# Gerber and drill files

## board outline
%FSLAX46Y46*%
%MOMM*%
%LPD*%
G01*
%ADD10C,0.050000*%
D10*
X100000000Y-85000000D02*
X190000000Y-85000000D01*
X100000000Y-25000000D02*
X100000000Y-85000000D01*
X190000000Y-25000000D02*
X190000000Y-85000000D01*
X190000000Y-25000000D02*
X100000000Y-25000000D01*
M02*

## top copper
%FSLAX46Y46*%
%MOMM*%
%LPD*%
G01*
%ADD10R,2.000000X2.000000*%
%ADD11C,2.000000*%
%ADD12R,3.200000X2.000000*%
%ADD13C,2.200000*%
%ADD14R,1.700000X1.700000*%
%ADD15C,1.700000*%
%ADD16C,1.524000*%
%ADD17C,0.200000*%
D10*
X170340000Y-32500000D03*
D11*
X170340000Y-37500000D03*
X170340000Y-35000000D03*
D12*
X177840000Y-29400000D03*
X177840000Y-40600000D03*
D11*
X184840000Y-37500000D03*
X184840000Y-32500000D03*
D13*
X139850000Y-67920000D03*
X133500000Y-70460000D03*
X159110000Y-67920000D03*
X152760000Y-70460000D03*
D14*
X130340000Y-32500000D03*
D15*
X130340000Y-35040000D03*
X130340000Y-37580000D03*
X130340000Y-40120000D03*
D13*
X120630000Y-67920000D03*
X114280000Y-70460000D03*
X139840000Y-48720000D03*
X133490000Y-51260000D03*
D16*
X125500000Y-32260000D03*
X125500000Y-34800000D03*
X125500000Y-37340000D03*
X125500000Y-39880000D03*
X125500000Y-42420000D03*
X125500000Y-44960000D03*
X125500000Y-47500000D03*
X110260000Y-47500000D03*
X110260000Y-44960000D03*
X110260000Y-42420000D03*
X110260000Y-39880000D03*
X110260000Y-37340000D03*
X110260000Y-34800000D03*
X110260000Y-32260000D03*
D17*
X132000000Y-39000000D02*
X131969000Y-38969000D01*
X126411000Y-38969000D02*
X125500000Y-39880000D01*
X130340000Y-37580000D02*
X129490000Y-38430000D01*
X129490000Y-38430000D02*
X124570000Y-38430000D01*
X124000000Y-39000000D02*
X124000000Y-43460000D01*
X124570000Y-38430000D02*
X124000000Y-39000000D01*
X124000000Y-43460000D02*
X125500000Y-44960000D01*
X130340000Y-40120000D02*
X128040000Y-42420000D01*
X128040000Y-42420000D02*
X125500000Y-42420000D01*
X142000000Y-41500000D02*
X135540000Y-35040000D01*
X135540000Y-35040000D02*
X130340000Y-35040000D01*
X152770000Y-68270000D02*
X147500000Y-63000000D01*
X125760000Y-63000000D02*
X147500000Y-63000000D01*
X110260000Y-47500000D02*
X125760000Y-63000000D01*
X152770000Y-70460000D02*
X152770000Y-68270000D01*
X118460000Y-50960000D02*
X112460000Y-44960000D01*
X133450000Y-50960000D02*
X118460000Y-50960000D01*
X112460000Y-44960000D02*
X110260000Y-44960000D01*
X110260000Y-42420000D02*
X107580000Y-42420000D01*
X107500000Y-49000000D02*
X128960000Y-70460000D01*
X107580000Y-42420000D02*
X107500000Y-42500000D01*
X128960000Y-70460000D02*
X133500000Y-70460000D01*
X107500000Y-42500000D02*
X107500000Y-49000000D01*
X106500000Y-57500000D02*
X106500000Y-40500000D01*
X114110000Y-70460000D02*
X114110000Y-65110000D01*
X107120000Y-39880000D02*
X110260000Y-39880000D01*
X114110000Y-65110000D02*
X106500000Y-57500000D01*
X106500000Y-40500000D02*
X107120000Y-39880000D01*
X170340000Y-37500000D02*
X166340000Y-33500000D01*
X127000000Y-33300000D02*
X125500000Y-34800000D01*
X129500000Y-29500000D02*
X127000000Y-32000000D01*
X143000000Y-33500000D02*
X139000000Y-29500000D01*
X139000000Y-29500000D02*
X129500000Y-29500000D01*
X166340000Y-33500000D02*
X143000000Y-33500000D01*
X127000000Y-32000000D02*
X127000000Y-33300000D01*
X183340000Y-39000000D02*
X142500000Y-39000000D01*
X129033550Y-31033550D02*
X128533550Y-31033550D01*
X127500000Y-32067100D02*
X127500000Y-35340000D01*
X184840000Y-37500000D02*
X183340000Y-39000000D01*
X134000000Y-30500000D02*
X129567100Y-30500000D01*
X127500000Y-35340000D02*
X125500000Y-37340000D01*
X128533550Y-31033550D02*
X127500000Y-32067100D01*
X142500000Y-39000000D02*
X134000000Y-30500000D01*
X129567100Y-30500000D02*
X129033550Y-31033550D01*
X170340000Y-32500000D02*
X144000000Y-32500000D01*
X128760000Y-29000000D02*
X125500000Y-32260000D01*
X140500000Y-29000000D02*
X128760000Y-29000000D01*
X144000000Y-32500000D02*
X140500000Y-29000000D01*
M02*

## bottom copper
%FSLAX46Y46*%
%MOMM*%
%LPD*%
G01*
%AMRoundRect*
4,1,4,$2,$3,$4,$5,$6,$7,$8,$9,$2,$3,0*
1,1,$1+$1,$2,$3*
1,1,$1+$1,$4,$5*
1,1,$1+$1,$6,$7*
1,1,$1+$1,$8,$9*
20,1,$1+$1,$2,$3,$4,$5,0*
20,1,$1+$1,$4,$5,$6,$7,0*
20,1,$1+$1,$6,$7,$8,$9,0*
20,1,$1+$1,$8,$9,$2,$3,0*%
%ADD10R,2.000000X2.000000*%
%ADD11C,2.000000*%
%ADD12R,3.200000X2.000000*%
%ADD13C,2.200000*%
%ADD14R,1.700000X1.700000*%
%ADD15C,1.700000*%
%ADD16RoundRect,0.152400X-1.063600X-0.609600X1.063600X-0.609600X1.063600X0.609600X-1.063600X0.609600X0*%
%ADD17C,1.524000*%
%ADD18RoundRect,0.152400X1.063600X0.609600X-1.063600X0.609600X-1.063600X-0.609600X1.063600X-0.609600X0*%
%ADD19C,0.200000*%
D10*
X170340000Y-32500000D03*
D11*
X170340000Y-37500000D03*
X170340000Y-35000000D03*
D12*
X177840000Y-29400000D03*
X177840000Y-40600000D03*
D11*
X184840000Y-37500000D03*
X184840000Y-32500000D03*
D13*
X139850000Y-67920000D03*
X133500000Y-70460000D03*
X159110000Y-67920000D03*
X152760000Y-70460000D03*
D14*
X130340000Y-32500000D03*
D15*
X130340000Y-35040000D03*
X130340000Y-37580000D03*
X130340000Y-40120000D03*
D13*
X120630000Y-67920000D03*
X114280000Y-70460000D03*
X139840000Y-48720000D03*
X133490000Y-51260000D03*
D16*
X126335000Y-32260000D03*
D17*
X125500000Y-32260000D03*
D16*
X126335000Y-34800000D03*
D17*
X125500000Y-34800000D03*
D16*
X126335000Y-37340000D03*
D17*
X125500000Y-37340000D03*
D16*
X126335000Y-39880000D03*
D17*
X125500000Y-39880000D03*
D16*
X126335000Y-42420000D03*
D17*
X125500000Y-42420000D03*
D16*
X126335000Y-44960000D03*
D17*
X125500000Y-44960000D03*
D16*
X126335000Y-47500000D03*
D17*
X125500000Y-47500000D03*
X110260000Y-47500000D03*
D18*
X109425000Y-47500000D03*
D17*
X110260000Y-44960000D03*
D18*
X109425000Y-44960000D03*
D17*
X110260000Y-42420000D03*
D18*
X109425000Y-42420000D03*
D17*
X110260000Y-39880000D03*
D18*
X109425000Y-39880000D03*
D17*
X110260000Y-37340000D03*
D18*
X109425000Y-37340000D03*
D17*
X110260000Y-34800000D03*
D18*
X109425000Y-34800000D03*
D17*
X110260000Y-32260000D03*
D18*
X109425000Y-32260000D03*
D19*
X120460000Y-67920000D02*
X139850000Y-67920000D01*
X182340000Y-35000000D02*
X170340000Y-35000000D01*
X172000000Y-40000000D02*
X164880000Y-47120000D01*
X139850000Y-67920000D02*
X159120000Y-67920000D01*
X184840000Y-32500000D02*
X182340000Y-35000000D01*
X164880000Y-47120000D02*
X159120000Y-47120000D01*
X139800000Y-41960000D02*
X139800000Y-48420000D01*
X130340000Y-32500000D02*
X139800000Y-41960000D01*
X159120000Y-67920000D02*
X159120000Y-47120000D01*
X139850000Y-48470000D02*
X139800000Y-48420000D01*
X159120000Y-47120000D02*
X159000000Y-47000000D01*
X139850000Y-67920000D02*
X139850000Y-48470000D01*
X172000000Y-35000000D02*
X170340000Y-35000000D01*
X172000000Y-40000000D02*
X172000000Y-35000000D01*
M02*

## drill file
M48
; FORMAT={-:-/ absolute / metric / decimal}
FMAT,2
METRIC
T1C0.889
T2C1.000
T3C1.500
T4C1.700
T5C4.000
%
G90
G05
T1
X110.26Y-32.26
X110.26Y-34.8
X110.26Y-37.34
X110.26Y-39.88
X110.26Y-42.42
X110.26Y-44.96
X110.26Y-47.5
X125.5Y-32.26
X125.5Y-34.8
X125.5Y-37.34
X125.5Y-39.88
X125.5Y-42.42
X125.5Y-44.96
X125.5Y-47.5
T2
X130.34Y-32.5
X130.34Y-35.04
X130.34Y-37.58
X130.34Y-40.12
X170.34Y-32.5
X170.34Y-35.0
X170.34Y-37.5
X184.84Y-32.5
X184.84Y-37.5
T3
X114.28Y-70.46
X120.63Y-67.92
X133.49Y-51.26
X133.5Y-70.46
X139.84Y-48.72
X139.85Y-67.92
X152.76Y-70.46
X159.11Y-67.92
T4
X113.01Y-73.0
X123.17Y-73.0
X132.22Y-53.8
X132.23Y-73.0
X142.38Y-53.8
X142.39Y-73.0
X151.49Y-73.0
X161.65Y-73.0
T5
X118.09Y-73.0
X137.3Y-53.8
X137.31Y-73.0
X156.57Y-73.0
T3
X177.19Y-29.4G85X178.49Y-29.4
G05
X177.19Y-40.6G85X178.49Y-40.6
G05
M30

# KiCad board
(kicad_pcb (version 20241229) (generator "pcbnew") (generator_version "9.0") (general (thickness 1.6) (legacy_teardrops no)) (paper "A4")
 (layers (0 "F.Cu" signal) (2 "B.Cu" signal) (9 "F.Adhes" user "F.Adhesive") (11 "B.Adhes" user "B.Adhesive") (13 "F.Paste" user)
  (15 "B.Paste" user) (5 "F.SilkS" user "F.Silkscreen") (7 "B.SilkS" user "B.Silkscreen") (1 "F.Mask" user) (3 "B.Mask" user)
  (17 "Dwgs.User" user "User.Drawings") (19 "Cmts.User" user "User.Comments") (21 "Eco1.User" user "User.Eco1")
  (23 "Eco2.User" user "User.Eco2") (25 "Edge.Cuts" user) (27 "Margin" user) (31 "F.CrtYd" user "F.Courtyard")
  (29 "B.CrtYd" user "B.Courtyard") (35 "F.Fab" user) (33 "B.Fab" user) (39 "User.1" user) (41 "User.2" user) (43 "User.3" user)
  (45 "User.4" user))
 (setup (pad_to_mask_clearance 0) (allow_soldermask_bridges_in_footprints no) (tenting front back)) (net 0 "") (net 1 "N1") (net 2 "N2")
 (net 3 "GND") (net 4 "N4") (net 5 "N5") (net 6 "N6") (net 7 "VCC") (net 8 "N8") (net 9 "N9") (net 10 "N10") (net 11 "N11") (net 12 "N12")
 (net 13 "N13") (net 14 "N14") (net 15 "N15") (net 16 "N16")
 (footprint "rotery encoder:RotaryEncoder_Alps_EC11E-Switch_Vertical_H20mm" (layer "F.Cu") (at 170.34 32.5)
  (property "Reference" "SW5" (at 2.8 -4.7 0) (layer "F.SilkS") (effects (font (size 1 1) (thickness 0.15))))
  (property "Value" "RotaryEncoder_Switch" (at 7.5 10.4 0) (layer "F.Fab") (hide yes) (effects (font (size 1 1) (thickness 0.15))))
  (pad "A" thru_hole rect (at 0 0) (size 2 2) (drill 1) (layers "*.Cu" "*.Mask") (remove_unused_layers no) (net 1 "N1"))
  (pad "B" thru_hole circle (at 0 5) (size 2 2) (drill 1) (layers "*.Cu" "*.Mask") (remove_unused_layers no) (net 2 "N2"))
  (pad "C" thru_hole circle (at 0 2.5) (size 2 2) (drill 1) (layers "*.Cu" "*.Mask") (remove_unused_layers no) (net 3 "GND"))
  (pad "MP" thru_hole rect (at 7.5 -3.1) (size 3.2 2) (drill oval 2.8 1.5) (layers "*.Cu" "*.Mask") (remove_unused_layers no))
  (pad "MP" thru_hole rect (at 7.5 8.1) (size 3.2 2) (drill oval 2.8 1.5) (layers "*.Cu" "*.Mask") (remove_unused_layers no))
  (pad "S1" thru_hole circle (at 14.5 5) (size 2 2) (drill 1) (layers "*.Cu" "*.Mask") (remove_unused_layers no) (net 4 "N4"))
  (pad "S2" thru_hole circle (at 14.5 0) (size 2 2) (drill 1) (layers "*.Cu" "*.Mask") (remove_unused_layers no) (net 3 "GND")))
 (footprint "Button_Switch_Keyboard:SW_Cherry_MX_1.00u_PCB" (layer "F.Cu") (at 139.85 67.92)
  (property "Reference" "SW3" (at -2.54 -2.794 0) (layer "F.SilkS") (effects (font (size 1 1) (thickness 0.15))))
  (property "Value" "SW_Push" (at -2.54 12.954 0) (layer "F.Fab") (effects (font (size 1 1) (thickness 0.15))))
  (pad "" np_thru_hole circle (at -7.62 5.08) (size 1.7 1.7) (drill 1.7) (layers "*.Cu" "*.Mask"))
  (pad "" np_thru_hole circle (at -2.54 5.08) (size 4 4) (drill 4) (layers "*.Cu" "*.Mask"))
  (pad "" np_thru_hole circle (at 2.54 5.08) (size 1.7 1.7) (drill 1.7) (layers "*.Cu" "*.Mask"))
  (pad "1" thru_hole circle (at 0 0) (size 2.2 2.2) (drill 1.5) (layers "*.Cu" "*.Mask") (remove_unused_layers no) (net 3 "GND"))
  (pad "2" thru_hole circle (at -6.35 2.54) (size 2.2 2.2) (drill 1.5) (layers "*.Cu" "*.Mask") (remove_unused_layers no) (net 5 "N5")))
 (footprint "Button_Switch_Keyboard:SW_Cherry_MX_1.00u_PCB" (layer "F.Cu") (at 159.11 67.92)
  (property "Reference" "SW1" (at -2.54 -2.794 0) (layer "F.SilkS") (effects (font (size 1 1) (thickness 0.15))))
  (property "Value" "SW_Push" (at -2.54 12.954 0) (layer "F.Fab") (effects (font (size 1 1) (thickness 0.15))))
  (pad "" np_thru_hole circle (at -7.62 5.08) (size 1.7 1.7) (drill 1.7) (layers "*.Cu" "*.Mask"))
  (pad "" np_thru_hole circle (at -2.54 5.08) (size 4 4) (drill 4) (layers "*.Cu" "*.Mask"))
  (pad "" np_thru_hole circle (at 2.54 5.08) (size 1.7 1.7) (drill 1.7) (layers "*.Cu" "*.Mask"))
  (pad "1" thru_hole circle (at 0 0) (size 2.2 2.2) (drill 1.5) (layers "*.Cu" "*.Mask") (remove_unused_layers no) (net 3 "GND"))
  (pad "2" thru_hole circle (at -6.35 2.54) (size 2.2 2.2) (drill 1.5) (layers "*.Cu" "*.Mask") (remove_unused_layers no) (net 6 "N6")))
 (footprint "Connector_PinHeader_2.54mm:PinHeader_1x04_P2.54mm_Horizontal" (layer "F.Cu") (at 130.34 32.5)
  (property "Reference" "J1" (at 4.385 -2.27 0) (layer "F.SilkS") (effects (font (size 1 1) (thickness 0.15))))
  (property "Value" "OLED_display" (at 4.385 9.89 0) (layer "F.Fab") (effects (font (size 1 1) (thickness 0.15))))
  (pad "1" thru_hole rect (at 0 0) (size 1.7 1.7) (drill 1) (layers "*.Cu" "*.Mask") (remove_unused_layers no) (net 3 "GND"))
  (pad "2" thru_hole circle (at 0 2.54) (size 1.7 1.7) (drill 1) (layers "*.Cu" "*.Mask") (remove_unused_layers no) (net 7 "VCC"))
  (pad "3" thru_hole circle (at 0 5.08) (size 1.7 1.7) (drill 1) (layers "*.Cu" "*.Mask") (remove_unused_layers no) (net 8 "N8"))
  (pad "4" thru_hole circle (at 0 7.62) (size 1.7 1.7) (drill 1) (layers "*.Cu" "*.Mask") (remove_unused_layers no) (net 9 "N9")))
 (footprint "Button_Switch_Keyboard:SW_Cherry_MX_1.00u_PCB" (layer "F.Cu") (at 120.63 67.92)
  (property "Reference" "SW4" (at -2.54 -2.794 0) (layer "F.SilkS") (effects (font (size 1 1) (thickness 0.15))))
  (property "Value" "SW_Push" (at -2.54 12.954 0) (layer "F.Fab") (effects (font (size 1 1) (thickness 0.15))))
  (pad "" np_thru_hole circle (at -7.62 5.08) (size 1.7 1.7) (drill 1.7) (layers "*.Cu" "*.Mask"))
  (pad "" np_thru_hole circle (at -2.54 5.08) (size 4 4) (drill 4) (layers "*.Cu" "*.Mask"))
  (pad "" np_thru_hole circle (at 2.54 5.08) (size 1.7 1.7) (drill 1.7) (layers "*.Cu" "*.Mask"))
  (pad "1" thru_hole circle (at 0 0) (size 2.2 2.2) (drill 1.5) (layers "*.Cu" "*.Mask") (remove_unused_layers no) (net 3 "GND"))
  (pad "2" thru_hole circle (at -6.35 2.54) (size 2.2 2.2) (drill 1.5) (layers "*.Cu" "*.Mask") (remove_unused_layers no) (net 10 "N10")))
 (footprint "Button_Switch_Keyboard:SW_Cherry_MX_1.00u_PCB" (layer "F.Cu") (at 139.84 48.72)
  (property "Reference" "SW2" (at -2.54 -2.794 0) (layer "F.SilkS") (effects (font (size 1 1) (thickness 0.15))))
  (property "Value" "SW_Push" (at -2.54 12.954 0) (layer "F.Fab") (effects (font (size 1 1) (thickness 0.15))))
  (pad "" np_thru_hole circle (at -7.62 5.08) (size 1.7 1.7) (drill 1.7) (layers "*.Cu" "*.Mask"))
  (pad "" np_thru_hole circle (at -2.54 5.08) (size 4 4) (drill 4) (layers "*.Cu" "*.Mask"))
  (pad "" np_thru_hole circle (at 2.54 5.08) (size 1.7 1.7) (drill 1.7) (layers "*.Cu" "*.Mask"))
  (pad "1" thru_hole circle (at 0 0) (size 2.2 2.2) (drill 1.5) (layers "*.Cu" "*.Mask") (remove_unused_layers no) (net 3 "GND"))
  (pad "2" thru_hole circle (at -6.35 2.54) (size 2.2 2.2) (drill 1.5) (layers "*.Cu" "*.Mask") (remove_unused_layers no) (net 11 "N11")))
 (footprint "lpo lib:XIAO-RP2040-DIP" (layer "B.Cu") (at 117.88 39.88 180)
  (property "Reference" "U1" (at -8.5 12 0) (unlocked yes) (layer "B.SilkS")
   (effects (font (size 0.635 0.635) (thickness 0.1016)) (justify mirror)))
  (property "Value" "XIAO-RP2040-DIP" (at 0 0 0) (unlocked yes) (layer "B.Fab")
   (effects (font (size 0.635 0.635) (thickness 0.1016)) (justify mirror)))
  (pad "1" smd roundrect (at -8.455 7.62) (size 2.432 1.524) (layers "B.Cu" "B.Mask") (roundrect_rratio 0.1) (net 1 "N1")
   (thermal_bridge_angle 45))
  (pad "1" thru_hole circle (at -7.62 7.62) (size 1.524 1.524) (drill 0.889) (layers "*.Cu" "*.Mask") (remove_unused_layers no) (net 1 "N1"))
  (pad "2" smd roundrect (at -8.455 5.08) (size 2.432 1.524) (layers "B.Cu" "B.Mask") (roundrect_rratio 0.1) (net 2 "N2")
   (thermal_bridge_angle 45))
  (pad "2" thru_hole circle (at -7.62 5.08) (size 1.524 1.524) (drill 0.889) (layers "*.Cu" "*.Mask") (remove_unused_layers no) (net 2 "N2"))
  (pad "3" smd roundrect (at -8.455 2.54) (size 2.432 1.524) (layers "B.Cu" "B.Mask") (roundrect_rratio 0.1) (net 4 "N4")
   (thermal_bridge_angle 45))
  (pad "3" thru_hole circle (at -7.62 2.54) (size 1.524 1.524) (drill 0.889) (layers "*.Cu" "*.Mask") (remove_unused_layers no) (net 4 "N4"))
  (pad "4" smd roundrect (at -8.455 0) (size 2.432 1.524) (layers "B.Cu" "B.Mask") (roundrect_rratio 0.1) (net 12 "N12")
   (thermal_bridge_angle 45))
  (pad "4" thru_hole circle (at -7.62 0) (size 1.524 1.524) (drill 0.889) (layers "*.Cu" "*.Mask") (remove_unused_layers no) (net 12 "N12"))
  (pad "5" smd roundrect (at -8.455 -2.54) (size 2.432 1.524) (layers "B.Cu" "B.Mask") (roundrect_rratio 0.1) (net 9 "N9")
   (thermal_bridge_angle 45))
  (pad "5" thru_hole circle (at -7.62 -2.54) (size 1.524 1.524) (drill 0.889) (layers "*.Cu" "*.Mask") (remove_unused_layers no)
   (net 9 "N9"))
  (pad "6" smd roundrect (at -8.455 -5.08) (size 2.432 1.524) (layers "B.Cu" "B.Mask") (roundrect_rratio 0.1) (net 8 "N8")
   (thermal_bridge_angle 45))
  (pad "6" thru_hole circle (at -7.62 -5.08) (size 1.524 1.524) (drill 0.889) (layers "*.Cu" "*.Mask") (remove_unused_layers no)
   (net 8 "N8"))
  (pad "7" smd roundrect (at -8.455 -7.62) (size 2.432 1.524) (layers "B.Cu" "B.Mask") (roundrect_rratio 0.1) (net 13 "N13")
   (thermal_bridge_angle 45))
  (pad "7" thru_hole circle (at -7.62 -7.62) (size 1.524 1.524) (drill 0.889) (layers "*.Cu" "*.Mask") (remove_unused_layers no)
   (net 13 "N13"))
  (pad "8" thru_hole circle (at 7.62 -7.62 180) (size 1.524 1.524) (drill 0.889) (layers "*.Cu" "*.Mask") (remove_unused_layers no)
   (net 6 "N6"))
  (pad "8" smd roundrect (at 8.455 -7.62 180) (size 2.432 1.524) (layers "B.Cu" "B.Mask") (roundrect_rratio 0.1) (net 6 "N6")
   (thermal_bridge_angle 45))
  (pad "9" thru_hole circle (at 7.62 -5.08 180) (size 1.524 1.524) (drill 0.889) (layers "*.Cu" "*.Mask") (remove_unused_layers no)
   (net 11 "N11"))
  (pad "9" smd roundrect (at 8.455 -5.08 180) (size 2.432 1.524) (layers "B.Cu" "B.Mask") (roundrect_rratio 0.1) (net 11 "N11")
   (thermal_bridge_angle 45))
  (pad "10" thru_hole circle (at 7.62 -2.54 180) (size 1.524 1.524) (drill 0.889) (layers "*.Cu" "*.Mask") (remove_unused_layers no)
   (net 5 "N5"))
  (pad "10" smd roundrect (at 8.455 -2.54 180) (size 2.432 1.524) (layers "B.Cu" "B.Mask") (roundrect_rratio 0.1) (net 5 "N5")
   (thermal_bridge_angle 45))
  (pad "11" thru_hole circle (at 7.62 0 180) (size 1.524 1.524) (drill 0.889) (layers "*.Cu" "*.Mask") (remove_unused_layers no)
   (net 10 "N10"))
  (pad "11" smd roundrect (at 8.455 0 180) (size 2.432 1.524) (layers "B.Cu" "B.Mask") (roundrect_rratio 0.1) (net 10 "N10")
   (thermal_bridge_angle 45))
  (pad "12" thru_hole circle (at 7.62 2.54 180) (size 1.524 1.524) (drill 0.889) (layers "*.Cu" "*.Mask") (remove_unused_layers no)
   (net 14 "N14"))
  (pad "12" smd roundrect (at 8.455 2.54 180) (size 2.432 1.524) (layers "B.Cu" "B.Mask") (roundrect_rratio 0.1) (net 14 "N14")
   (thermal_bridge_angle 45))
  (pad "13" thru_hole circle (at 7.62 5.08 180) (size 1.524 1.524) (drill 0.889) (layers "*.Cu" "*.Mask") (remove_unused_layers no)
   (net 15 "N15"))
  (pad "13" smd roundrect (at 8.455 5.08 180) (size 2.432 1.524) (layers "B.Cu" "B.Mask") (roundrect_rratio 0.1) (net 15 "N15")
   (thermal_bridge_angle 45))
  (pad "14" thru_hole circle (at 7.62 7.62 180) (size 1.524 1.524) (drill 0.889) (layers "*.Cu" "*.Mask") (remove_unused_layers no)
   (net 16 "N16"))
  (pad "14" smd roundrect (at 8.455 7.62 180) (size 2.432 1.524) (layers "B.Cu" "B.Mask") (roundrect_rratio 0.1) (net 16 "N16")
   (thermal_bridge_angle 45)))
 (gr_line (start 100 85) (end 190 85) (stroke (width 0.05) (type default)) (layer "Edge.Cuts"))
 (gr_line (start 100 25) (end 100 85) (stroke (width 0.05) (type default)) (layer "Edge.Cuts"))
 (gr_line (start 190 25) (end 190 85) (stroke (width 0.05) (type default)) (layer "Edge.Cuts"))
 (gr_line (start 190 25) (end 100 25) (stroke (width 0.05) (type default)) (layer "Edge.Cuts"))
 (segment (start 132 39) (end 131.969 38.969) (width 0.2) (layer "F.Cu") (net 12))
 (segment (start 126.411 38.969) (end 125.5 39.88) (width 0.2) (layer "F.Cu") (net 12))
 (segment (start 120.46 67.92) (end 139.85 67.92) (width 0.2) (layer "B.Cu") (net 3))
 (segment (start 182.34 35) (end 170.34 35) (width 0.2) (layer "B.Cu") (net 3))
 (segment (start 172 40) (end 164.88 47.12) (width 0.2) (layer "B.Cu") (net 3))
 (segment (start 139.85 67.92) (end 159.12 67.92) (width 0.2) (layer "B.Cu") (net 3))
 (segment (start 184.84 32.5) (end 182.34 35) (width 0.2) (layer "B.Cu") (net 3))
 (segment (start 164.88 47.12) (end 159.12 47.12) (width 0.2) (layer "B.Cu") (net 3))
 (segment (start 139.8 41.96) (end 139.8 48.42) (width 0.2) (layer "B.Cu") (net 3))
 (segment (start 130.34 32.5) (end 139.8 41.96) (width 0.2) (layer "B.Cu") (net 3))
 (segment (start 159.12 67.92) (end 159.12 47.12) (width 0.2) (layer "B.Cu") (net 3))
 (segment (start 139.85 48.47) (end 139.8 48.42) (width 0.2) (layer "B.Cu") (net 3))
 (segment (start 159.12 47.12) (end 159 47) (width 0.2) (layer "B.Cu") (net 3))
 (segment (start 139.85 67.92) (end 139.85 48.47) (width 0.2) (layer "B.Cu") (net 3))
 (segment (start 172 35) (end 170.34 35) (width 0.2) (layer "B.Cu") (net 3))
 (segment (start 172 40) (end 172 35) (width 0.2) (layer "B.Cu") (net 3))
 (segment (start 130.34 37.58) (end 129.49 38.43) (width 0.2) (layer "F.Cu") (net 8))
 (segment (start 129.49 38.43) (end 124.57 38.43) (width 0.2) (layer "F.Cu") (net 8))
 (segment (start 124 39) (end 124 43.46) (width 0.2) (layer "F.Cu") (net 8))
 (segment (start 124.57 38.43) (end 124 39) (width 0.2) (layer "F.Cu") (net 8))
 (segment (start 124 43.46) (end 125.5 44.96) (width 0.2) (layer "F.Cu") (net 8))
 (segment (start 130.34 40.12) (end 128.04 42.42) (width 0.2) (layer "F.Cu") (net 9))
 (segment (start 128.04 42.42) (end 125.5 42.42) (width 0.2) (layer "F.Cu") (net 9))
 (segment (start 142 41.5) (end 135.54 35.04) (width 0.2) (layer "F.Cu") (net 7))
 (segment (start 135.54 35.04) (end 130.34 35.04) (width 0.2) (layer "F.Cu") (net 7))
 (segment (start 152.77 68.27) (end 147.5 63) (width 0.2) (layer "F.Cu") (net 6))
 (segment (start 125.76 63) (end 147.5 63) (width 0.2) (layer "F.Cu") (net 6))
 (segment (start 110.26 47.5) (end 125.76 63) (width 0.2) (layer "F.Cu") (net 6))
 (segment (start 152.77 70.46) (end 152.77 68.27) (width 0.2) (layer "F.Cu") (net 6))
 (segment (start 118.46 50.96) (end 112.46 44.96) (width 0.2) (layer "F.Cu") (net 11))
 (segment (start 133.45 50.96) (end 118.46 50.96) (width 0.2) (layer "F.Cu") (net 11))
 (segment (start 112.46 44.96) (end 110.26 44.96) (width 0.2) (layer "F.Cu") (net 11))
 (segment (start 110.26 42.42) (end 107.58 42.42) (width 0.2) (layer "F.Cu") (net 5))
 (segment (start 107.5 49) (end 128.96 70.46) (width 0.2) (layer "F.Cu") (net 5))
 (segment (start 107.58 42.42) (end 107.5 42.5) (width 0.2) (layer "F.Cu") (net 5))
 (segment (start 128.96 70.46) (end 133.5 70.46) (width 0.2) (layer "F.Cu") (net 5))
 (segment (start 107.5 42.5) (end 107.5 49) (width 0.2) (layer "F.Cu") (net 5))
 (segment (start 106.5 57.5) (end 106.5 40.5) (width 0.2) (layer "F.Cu") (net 10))
 (segment (start 114.11 70.46) (end 114.11 65.11) (width 0.2) (layer "F.Cu") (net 10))
 (segment (start 107.12 39.88) (end 110.26 39.88) (width 0.2) (layer "F.Cu") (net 10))
 (segment (start 114.11 65.11) (end 106.5 57.5) (width 0.2) (layer "F.Cu") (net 10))
 (segment (start 106.5 40.5) (end 107.12 39.88) (width 0.2) (layer "F.Cu") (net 10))
 (segment (start 170.34 37.5) (end 166.34 33.5) (width 0.2) (layer "F.Cu") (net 2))
 (segment (start 127 33.3) (end 125.5 34.8) (width 0.2) (layer "F.Cu") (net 2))
 (segment (start 129.5 29.5) (end 127 32) (width 0.2) (layer "F.Cu") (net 2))
 (segment (start 143 33.5) (end 139 29.5) (width 0.2) (layer "F.Cu") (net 2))
 (segment (start 139 29.5) (end 129.5 29.5) (width 0.2) (layer "F.Cu") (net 2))
 (segment (start 166.34 33.5) (end 143 33.5) (width 0.2) (layer "F.Cu") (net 2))
 (segment (start 127 32) (end 127 33.3) (width 0.2) (layer "F.Cu") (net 2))
 (segment (start 183.34 39) (end 142.5 39) (width 0.2) (layer "F.Cu") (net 4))
 (segment (start 129.03355 31.03355) (end 128.53355 31.03355) (width 0.2) (layer "F.Cu") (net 4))
 (segment (start 127.5 32.0671) (end 127.5 35.34) (width 0.2) (layer "F.Cu") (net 4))
 (segment (start 184.84 37.5) (end 183.34 39) (width 0.2) (layer "F.Cu") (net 4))
 (segment (start 134 30.5) (end 129.5671 30.5) (width 0.2) (layer "F.Cu") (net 4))
 (segment (start 127.5 35.34) (end 125.5 37.34) (width 0.2) (layer "F.Cu") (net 4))
 (segment (start 128.53355 31.03355) (end 127.5 32.0671) (width 0.2) (layer "F.Cu") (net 4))
 (segment (start 142.5 39) (end 134 30.5) (width 0.2) (layer "F.Cu") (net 4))
 (segment (start 129.5671 30.5) (end 129.03355 31.03355) (width 0.2) (layer "F.Cu") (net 4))
 (segment (start 170.34 32.5) (end 144 32.5) (width 0.2) (layer "F.Cu") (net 1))
 (segment (start 128.76 29) (end 125.5 32.26) (width 0.2) (layer "F.Cu") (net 1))
 (segment (start 140.5 29) (end 128.76 29) (width 0.2) (layer "F.Cu") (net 1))
 (segment (start 144 32.5) (end 140.5 29) (width 0.2) (layer "F.Cu") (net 1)))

